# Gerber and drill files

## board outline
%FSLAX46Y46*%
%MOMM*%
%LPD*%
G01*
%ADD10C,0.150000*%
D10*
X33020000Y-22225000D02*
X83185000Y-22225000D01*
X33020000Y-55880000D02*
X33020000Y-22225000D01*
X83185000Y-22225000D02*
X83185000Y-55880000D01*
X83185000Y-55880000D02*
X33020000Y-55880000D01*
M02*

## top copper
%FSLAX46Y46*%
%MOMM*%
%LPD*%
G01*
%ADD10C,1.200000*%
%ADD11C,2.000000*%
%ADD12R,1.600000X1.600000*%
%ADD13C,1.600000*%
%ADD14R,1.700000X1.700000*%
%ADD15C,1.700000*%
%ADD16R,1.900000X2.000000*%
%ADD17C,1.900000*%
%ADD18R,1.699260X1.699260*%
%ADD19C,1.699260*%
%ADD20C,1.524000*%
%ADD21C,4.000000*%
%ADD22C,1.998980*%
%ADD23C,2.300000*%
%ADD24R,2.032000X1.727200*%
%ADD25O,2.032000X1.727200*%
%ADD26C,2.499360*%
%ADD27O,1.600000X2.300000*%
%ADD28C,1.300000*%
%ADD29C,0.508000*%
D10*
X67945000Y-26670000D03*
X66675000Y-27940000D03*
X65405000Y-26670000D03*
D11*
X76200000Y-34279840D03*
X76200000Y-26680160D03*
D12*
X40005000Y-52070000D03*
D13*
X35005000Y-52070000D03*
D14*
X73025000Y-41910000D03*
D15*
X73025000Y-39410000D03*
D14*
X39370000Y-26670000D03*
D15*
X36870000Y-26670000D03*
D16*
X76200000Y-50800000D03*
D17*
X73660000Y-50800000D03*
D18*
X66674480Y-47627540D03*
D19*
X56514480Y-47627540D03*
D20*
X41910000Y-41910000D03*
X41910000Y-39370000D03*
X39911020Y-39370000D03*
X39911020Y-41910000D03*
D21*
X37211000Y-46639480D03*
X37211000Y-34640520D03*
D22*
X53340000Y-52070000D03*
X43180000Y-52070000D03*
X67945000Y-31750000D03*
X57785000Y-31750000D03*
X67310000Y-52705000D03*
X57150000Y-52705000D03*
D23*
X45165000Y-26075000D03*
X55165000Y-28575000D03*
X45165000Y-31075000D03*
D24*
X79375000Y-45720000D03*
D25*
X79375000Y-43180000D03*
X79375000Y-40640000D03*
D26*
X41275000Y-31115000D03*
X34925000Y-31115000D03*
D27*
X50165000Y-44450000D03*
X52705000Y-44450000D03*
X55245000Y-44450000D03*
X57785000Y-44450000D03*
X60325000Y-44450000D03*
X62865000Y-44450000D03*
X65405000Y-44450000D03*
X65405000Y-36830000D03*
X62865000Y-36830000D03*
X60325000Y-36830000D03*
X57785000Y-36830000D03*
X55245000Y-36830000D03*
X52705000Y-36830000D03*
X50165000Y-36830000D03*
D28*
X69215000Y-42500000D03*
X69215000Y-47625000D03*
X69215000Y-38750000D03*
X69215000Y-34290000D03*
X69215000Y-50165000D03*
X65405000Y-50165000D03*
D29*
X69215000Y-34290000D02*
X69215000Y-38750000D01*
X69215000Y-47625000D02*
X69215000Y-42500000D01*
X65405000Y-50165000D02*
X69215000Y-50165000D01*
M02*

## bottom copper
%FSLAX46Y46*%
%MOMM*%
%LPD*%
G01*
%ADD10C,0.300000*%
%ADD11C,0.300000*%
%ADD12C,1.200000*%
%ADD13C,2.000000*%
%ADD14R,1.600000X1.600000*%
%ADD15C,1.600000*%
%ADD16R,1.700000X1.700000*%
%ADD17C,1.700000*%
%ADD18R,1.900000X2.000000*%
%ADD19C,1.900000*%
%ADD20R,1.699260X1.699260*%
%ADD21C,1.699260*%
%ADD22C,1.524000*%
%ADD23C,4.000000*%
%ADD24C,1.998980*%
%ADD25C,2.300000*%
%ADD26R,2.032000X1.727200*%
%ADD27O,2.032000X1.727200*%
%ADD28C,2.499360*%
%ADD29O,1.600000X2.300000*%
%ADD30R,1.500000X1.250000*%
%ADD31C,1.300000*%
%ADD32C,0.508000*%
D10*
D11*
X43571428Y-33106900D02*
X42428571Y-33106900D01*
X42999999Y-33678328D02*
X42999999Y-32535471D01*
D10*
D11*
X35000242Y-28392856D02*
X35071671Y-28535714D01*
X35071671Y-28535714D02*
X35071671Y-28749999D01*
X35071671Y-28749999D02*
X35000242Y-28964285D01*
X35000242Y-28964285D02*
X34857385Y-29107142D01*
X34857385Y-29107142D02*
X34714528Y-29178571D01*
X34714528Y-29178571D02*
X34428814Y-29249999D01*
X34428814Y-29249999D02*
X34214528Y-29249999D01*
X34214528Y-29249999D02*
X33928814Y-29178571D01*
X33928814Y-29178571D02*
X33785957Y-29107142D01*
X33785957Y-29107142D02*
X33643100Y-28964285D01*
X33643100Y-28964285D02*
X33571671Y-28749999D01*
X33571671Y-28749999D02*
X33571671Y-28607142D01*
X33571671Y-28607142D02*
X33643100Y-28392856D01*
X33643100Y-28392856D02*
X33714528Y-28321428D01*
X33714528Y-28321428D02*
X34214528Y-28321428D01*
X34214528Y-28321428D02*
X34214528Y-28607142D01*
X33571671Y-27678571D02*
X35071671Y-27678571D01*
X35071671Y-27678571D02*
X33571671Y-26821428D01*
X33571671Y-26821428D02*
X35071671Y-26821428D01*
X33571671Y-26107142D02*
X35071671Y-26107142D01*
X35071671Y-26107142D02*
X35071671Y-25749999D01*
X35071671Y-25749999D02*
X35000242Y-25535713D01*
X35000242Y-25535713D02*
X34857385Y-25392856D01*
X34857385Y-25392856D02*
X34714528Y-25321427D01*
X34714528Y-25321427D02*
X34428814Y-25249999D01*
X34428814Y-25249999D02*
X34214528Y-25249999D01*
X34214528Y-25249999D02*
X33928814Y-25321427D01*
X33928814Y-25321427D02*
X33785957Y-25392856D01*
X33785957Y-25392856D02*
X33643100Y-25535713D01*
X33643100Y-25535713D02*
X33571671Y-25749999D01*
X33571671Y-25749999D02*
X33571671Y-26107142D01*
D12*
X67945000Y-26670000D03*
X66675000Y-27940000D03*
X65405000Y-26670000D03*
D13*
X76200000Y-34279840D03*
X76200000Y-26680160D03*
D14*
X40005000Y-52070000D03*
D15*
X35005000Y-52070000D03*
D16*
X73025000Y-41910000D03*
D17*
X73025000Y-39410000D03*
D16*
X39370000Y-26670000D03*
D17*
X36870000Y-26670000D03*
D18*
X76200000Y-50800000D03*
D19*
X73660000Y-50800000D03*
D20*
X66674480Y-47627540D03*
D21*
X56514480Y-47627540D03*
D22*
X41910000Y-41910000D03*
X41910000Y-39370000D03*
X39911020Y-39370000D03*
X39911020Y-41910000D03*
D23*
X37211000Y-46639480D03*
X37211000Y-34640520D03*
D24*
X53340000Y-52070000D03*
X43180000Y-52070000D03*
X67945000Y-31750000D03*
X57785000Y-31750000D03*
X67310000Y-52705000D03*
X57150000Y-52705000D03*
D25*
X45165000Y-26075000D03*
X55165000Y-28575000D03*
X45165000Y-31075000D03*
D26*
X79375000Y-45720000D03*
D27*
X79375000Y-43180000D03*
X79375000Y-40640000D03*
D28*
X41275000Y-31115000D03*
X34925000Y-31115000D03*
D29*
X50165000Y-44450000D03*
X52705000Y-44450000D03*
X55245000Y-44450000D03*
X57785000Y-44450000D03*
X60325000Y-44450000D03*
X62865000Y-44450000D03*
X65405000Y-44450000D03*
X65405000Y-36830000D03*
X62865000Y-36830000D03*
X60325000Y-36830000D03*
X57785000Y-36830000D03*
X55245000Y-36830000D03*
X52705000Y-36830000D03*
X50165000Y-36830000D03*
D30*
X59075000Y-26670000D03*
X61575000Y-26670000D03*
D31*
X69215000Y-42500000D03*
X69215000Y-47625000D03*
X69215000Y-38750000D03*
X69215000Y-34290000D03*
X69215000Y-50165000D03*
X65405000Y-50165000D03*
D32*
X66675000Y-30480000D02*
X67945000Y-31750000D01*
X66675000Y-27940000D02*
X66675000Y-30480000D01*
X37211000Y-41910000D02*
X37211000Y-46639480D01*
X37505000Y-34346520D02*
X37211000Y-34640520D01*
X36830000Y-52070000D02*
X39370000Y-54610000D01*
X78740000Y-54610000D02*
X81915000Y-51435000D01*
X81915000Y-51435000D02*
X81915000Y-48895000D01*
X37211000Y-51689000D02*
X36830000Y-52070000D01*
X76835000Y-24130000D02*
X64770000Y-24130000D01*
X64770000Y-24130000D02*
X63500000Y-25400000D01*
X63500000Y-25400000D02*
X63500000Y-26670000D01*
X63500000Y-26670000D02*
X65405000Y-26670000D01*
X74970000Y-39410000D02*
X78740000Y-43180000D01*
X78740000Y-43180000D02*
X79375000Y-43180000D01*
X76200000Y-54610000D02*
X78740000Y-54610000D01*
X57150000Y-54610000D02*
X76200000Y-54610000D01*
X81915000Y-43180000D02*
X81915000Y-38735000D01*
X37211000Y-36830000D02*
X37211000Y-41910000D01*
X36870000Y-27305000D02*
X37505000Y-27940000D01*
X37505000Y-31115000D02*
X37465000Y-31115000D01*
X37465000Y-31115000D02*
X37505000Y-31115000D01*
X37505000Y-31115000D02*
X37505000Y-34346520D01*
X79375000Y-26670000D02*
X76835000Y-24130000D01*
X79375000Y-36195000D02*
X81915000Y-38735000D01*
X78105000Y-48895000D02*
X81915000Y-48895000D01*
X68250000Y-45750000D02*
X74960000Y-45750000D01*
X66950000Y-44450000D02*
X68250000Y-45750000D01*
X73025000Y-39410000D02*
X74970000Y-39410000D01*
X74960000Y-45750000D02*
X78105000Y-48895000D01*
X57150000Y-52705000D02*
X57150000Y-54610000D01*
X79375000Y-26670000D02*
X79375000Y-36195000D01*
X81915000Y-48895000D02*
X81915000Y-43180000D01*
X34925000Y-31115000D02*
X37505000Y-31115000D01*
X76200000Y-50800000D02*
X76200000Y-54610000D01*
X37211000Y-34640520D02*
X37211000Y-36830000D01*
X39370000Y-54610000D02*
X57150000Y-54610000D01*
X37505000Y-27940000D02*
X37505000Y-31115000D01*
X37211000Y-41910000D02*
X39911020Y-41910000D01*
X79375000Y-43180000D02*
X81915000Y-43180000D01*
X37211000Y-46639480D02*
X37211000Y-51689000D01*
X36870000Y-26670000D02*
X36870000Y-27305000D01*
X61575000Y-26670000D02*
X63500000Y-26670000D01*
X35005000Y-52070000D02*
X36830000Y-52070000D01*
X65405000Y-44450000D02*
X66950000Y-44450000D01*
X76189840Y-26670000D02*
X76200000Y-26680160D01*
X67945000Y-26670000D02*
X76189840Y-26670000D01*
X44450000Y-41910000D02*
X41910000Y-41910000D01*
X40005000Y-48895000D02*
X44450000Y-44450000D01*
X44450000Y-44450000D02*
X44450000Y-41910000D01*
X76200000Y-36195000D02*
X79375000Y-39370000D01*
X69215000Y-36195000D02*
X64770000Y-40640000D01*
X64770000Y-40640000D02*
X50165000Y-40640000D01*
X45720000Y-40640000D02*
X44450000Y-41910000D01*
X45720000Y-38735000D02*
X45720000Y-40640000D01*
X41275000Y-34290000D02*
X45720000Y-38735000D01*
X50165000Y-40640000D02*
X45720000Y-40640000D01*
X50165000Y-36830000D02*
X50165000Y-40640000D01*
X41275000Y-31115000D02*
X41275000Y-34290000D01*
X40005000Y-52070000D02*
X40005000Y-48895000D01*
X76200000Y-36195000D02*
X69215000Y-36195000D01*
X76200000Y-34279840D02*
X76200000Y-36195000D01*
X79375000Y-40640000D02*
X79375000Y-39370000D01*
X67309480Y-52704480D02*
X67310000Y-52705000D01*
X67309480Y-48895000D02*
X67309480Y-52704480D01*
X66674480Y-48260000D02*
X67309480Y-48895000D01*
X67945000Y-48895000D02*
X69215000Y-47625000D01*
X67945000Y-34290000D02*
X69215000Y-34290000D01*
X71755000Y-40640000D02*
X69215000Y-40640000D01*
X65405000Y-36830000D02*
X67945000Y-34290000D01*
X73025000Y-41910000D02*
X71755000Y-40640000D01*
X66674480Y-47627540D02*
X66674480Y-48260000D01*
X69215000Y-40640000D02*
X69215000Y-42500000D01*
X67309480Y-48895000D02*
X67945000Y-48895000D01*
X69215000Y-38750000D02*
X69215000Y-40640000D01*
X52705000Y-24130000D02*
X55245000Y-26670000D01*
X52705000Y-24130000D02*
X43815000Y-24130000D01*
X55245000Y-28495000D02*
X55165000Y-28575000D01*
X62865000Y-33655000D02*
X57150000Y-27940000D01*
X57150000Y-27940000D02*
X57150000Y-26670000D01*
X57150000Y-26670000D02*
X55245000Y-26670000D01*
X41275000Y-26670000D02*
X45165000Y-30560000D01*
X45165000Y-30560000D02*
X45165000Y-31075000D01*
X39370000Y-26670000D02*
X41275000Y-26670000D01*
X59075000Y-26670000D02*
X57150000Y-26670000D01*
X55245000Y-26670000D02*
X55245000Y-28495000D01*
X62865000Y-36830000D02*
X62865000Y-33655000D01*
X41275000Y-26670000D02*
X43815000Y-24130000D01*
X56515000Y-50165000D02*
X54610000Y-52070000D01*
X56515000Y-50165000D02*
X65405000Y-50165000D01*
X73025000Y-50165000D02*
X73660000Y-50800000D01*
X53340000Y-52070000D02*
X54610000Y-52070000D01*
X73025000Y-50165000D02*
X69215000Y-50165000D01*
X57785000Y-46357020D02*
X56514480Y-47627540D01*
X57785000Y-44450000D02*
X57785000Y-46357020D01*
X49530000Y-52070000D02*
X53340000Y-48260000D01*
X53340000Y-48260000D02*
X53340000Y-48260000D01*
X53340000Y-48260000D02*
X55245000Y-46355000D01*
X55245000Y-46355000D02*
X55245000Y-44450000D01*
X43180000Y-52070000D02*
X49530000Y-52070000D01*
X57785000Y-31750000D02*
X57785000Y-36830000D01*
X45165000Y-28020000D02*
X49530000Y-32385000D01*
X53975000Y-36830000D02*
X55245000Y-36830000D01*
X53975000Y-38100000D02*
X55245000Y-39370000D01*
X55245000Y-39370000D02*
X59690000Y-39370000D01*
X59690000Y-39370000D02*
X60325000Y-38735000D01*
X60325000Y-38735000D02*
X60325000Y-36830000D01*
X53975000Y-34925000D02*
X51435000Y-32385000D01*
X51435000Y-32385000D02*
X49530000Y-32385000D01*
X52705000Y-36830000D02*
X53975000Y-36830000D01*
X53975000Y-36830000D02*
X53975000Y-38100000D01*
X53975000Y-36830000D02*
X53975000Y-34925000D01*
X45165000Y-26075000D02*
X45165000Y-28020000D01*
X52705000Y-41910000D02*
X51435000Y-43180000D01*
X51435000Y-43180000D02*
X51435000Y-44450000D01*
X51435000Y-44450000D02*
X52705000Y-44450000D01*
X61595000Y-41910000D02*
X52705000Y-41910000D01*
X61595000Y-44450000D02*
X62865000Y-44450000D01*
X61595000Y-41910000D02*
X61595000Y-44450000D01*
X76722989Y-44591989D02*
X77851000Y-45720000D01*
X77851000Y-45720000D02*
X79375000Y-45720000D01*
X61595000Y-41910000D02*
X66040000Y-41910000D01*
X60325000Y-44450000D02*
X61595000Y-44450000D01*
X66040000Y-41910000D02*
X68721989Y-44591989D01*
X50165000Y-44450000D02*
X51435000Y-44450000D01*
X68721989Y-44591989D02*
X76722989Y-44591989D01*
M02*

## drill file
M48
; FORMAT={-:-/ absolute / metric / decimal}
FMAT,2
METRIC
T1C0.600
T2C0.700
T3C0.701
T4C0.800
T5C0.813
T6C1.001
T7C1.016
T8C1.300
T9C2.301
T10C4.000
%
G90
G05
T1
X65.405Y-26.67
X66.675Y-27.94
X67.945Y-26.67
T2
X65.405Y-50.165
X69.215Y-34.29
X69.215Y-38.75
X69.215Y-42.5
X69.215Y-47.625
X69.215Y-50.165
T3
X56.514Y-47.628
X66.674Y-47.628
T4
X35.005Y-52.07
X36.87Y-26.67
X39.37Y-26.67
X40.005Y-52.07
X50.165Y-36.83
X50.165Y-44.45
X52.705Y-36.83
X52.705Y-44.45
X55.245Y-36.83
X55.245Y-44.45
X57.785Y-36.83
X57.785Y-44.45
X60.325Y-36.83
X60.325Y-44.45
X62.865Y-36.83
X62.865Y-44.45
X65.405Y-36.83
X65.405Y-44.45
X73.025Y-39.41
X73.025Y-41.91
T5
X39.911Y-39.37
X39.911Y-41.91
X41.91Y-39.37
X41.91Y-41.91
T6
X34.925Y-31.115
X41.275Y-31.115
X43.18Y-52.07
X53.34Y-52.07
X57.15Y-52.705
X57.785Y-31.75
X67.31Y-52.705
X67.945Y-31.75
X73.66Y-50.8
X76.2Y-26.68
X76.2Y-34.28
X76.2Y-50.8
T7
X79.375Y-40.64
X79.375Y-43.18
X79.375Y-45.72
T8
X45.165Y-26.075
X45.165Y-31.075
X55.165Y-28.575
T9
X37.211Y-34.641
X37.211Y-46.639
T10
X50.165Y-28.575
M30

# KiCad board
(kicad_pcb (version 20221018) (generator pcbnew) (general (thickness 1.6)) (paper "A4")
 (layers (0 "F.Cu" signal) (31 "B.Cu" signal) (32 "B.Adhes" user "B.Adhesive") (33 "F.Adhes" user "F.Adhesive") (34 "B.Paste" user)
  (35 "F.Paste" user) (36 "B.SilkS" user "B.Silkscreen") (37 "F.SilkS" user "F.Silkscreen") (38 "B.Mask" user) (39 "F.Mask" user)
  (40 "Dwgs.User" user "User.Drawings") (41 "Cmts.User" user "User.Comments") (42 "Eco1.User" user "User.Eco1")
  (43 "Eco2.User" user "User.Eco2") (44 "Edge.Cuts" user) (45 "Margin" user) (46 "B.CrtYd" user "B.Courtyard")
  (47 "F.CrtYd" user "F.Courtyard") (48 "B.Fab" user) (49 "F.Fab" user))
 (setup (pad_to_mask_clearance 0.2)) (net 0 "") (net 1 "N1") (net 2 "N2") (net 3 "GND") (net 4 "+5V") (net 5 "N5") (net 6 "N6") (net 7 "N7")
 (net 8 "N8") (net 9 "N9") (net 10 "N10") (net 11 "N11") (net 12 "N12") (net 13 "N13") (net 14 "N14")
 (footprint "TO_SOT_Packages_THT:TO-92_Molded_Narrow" (layer "F.Cu") (at 67.945 26.67 180)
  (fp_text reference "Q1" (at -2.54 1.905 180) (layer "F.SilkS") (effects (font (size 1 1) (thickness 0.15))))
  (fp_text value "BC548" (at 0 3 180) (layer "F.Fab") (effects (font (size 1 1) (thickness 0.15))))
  (pad "1" thru_hole circle (at 0 0 270) (size 1.2 1.2) (drill 0.6) (layers "*.Cu" "*.Mask" "F.SilkS") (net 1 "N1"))
  (pad "2" thru_hole circle (at 1.27 -1.27 270) (size 1.2 1.2) (drill 0.6) (layers "*.Cu" "*.Mask" "F.SilkS") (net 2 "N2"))
  (pad "3" thru_hole circle (at 2.54 0 270) (size 1.2 1.2) (drill 0.6) (layers "*.Cu" "*.Mask" "F.SilkS") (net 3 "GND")))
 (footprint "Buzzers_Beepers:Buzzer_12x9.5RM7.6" (layer "F.Cu") (at 76.2 30.48 90)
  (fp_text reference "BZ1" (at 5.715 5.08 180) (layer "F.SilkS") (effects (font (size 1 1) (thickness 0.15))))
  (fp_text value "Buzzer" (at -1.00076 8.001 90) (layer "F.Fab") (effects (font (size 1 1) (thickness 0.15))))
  (pad "1" thru_hole circle (at -3.79984 0 90) (size 2 2) (drill 1.00076) (layers "*.Cu" "*.Mask" "F.SilkS") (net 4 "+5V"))
  (pad "2" thru_hole circle (at 3.79984 0 90) (size 2 2) (drill 1.00076) (layers "*.Cu" "*.Mask" "F.SilkS") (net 1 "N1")))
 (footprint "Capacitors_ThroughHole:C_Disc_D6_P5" (layer "F.Cu") (at 40.005 52.07 180)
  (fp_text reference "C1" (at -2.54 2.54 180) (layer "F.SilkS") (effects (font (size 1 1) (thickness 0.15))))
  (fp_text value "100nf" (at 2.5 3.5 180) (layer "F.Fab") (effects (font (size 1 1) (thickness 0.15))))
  (pad "1" thru_hole rect (at 0 0 180) (size 1.6 1.6) (drill 0.8) (layers "*.Cu" "*.Mask" "F.SilkS") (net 4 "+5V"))
  (pad "2" thru_hole circle (at 5 0 180) (size 1.6 1.6) (drill 0.8) (layers "*.Cu" "*.Mask" "F.SilkS") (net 3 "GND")))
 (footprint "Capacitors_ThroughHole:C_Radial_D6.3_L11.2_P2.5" (layer "F.Cu") (at 73.025 41.91 90)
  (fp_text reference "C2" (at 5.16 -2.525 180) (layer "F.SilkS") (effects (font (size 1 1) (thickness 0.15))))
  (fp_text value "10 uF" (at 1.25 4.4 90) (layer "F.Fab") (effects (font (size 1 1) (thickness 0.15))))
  (pad "1" thru_hole rect (at 0 0 90) (size 1.7 1.7) (drill 0.8) (layers "*.Cu" "*.Mask" "F.SilkS") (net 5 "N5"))
  (pad "2" thru_hole circle (at 2.5 0 90) (size 1.7 1.7) (drill 0.8) (layers "*.Cu" "*.Mask" "F.SilkS") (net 3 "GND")))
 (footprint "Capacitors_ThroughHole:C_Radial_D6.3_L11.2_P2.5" (layer "F.Cu") (at 39.37 26.67 180)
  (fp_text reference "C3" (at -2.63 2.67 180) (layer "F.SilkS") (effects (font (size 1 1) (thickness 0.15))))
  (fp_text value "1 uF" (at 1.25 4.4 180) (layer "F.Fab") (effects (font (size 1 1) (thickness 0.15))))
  (pad "1" thru_hole rect (at 0 0 180) (size 1.7 1.7) (drill 0.8) (layers "*.Cu" "*.Mask" "F.SilkS") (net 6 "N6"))
  (pad "2" thru_hole circle (at 2.5 0 180) (size 1.7 1.7) (drill 0.8) (layers "*.Cu" "*.Mask" "F.SilkS") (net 3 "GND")))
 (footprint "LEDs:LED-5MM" (layer "F.Cu") (at 76.2 50.8 180)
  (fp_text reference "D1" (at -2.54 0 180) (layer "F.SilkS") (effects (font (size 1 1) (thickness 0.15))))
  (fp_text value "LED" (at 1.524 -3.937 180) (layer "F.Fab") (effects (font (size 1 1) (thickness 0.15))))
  (pad "1" thru_hole rect (at 0 0 270) (size 2 1.9) (drill 1.00076) (layers "*.Cu" "*.Mask" "F.SilkS") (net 3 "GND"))
  (pad "2" thru_hole circle (at 2.54 0 180) (size 1.9 1.9) (drill 1.00076) (layers "*.Cu" "*.Mask" "F.SilkS") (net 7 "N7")))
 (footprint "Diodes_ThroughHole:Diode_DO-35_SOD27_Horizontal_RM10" (layer "F.Cu") (at 66.675 47.625 180)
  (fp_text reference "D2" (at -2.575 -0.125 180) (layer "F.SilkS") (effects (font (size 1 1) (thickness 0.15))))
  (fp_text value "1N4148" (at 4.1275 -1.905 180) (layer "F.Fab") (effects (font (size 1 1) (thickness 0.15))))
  (pad "1" thru_hole rect (at 0.00052 -0.00254) (size 1.69926 1.69926) (drill 0.70104) (layers "*.Cu" "*.Mask" "F.SilkS") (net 5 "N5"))
  (pad "2" thru_hole circle (at 10.16052 -0.00254) (size 1.69926 1.69926) (drill 0.70104) (layers "*.Cu" "*.Mask" "F.SilkS") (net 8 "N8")))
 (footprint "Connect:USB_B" (layer "F.Cu") (at 41.91 41.91 180) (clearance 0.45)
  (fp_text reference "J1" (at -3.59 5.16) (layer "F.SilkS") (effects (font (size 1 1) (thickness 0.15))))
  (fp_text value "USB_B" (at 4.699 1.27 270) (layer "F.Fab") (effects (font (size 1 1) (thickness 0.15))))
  (pad "1" thru_hole circle (at 0 0 90) (size 1.524 1.524) (drill 0.8128) (layers "*.Cu" "*.Mask" "F.SilkS") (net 4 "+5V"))
  (pad "2" thru_hole circle (at 0 2.54 90) (size 1.524 1.524) (drill 0.8128) (layers "*.Cu" "*.Mask" "F.SilkS") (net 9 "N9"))
  (pad "3" thru_hole circle (at 1.99898 2.54 90) (size 1.524 1.524) (drill 0.8128) (layers "*.Cu" "*.Mask" "F.SilkS") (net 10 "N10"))
  (pad "4" thru_hole circle (at 1.99898 0 90) (size 1.524 1.524) (drill 0.8128) (layers "*.Cu" "*.Mask" "F.SilkS") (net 3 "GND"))
  (pad "5" thru_hole circle (at 4.699 -4.72948 90) (size 4 4) (drill 2.30124) (layers "*.Cu" "*.Mask" "F.SilkS") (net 3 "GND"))
  (pad "5" thru_hole circle (at 4.699 7.26948 90) (size 4 4) (drill 2.30124) (layers "*.Cu" "*.Mask" "F.SilkS") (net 3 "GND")))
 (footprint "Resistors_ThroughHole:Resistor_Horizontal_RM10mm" (layer "F.Cu") (at 53.34 52.07 180)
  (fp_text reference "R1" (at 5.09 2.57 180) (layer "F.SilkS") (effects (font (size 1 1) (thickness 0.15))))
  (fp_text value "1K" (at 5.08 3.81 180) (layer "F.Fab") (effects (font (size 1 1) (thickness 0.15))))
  (pad "1" thru_hole circle (at 0 0 180) (size 1.99898 1.99898) (drill 1.00076) (layers "*.Cu" "*.SilkS" "*.Mask") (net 7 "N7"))
  (pad "2" thru_hole circle (at 10.16 0 180) (size 1.99898 1.99898) (drill 1.00076) (layers "*.Cu" "*.SilkS" "*.Mask") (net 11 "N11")))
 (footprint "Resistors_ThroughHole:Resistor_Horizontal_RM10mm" (layer "F.Cu") (at 67.945 31.75 180)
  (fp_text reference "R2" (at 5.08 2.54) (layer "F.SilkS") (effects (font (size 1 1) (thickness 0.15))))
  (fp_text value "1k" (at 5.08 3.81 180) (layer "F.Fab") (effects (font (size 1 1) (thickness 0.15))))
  (pad "1" thru_hole circle (at 0 0 180) (size 1.99898 1.99898) (drill 1.00076) (layers "*.Cu" "*.SilkS" "*.Mask") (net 2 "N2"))
  (pad "2" thru_hole circle (at 10.16 0 180) (size 1.99898 1.99898) (drill 1.00076) (layers "*.Cu" "*.SilkS" "*.Mask") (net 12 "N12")))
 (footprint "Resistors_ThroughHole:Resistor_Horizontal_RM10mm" (layer "F.Cu") (at 67.31 52.705 180)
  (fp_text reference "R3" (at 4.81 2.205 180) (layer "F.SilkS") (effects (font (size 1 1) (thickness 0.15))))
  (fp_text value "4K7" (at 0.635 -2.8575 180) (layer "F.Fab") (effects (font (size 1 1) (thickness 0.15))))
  (pad "1" thru_hole circle (at 0 0 180) (size 1.99898 1.99898) (drill 1.00076) (layers "*.Cu" "*.SilkS" "*.Mask") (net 5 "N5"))
  (pad "2" thru_hole circle (at 10.16 0 180) (size 1.99898 1.99898) (drill 1.00076) (layers "*.Cu" "*.SilkS" "*.Mask") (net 3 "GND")))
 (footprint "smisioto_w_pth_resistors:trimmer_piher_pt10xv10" (layer "F.Cu") (at 50.165 28.575 90)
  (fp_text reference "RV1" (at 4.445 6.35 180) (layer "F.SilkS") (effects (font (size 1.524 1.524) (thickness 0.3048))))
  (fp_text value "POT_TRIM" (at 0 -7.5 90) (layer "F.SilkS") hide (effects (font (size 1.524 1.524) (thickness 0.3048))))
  (pad "" np_thru_hole circle (at 0 0 90) (size 4 4) (drill 4) (layers "*.Cu" "*.Mask" "F.SilkS"))
  (pad "1" thru_hole circle (at 2.5 -5 90) (size 2.3 2.3) (drill 1.3) (layers "*.Cu" "*.Mask" "F.SilkS") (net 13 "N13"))
  (pad "2" thru_hole circle (at 0 5 90) (size 2.3 2.3) (drill 1.3) (layers "*.Cu" "*.Mask" "F.SilkS") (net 6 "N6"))
  (pad "3" thru_hole circle (at -2.5 -5 90) (size 2.3 2.3) (drill 1.3) (layers "*.Cu" "*.Mask" "F.SilkS") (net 6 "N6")))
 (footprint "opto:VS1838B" (layer "F.Cu") (at 79.375 45.72 180)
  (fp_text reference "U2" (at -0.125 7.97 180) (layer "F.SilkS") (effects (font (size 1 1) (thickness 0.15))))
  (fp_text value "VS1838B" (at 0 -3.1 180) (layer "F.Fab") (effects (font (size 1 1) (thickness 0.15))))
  (pad "1" thru_hole rect (at 0 0 180) (size 2.032 1.7272) (drill 1.016) (layers "*.Cu" "*.Mask" "F.SilkS") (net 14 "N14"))
  (pad "2" thru_hole oval (at 0 2.54 180) (size 2.032 1.7272) (drill 1.016) (layers "*.Cu" "*.Mask" "F.SilkS") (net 3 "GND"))
  (pad "3" thru_hole oval (at 0 5.08 180) (size 2.032 1.7272) (drill 1.016) (layers "*.Cu" "*.Mask" "F.SilkS") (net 4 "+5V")))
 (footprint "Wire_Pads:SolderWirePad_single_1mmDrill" (layer "F.Cu") (at 41.275 31.115)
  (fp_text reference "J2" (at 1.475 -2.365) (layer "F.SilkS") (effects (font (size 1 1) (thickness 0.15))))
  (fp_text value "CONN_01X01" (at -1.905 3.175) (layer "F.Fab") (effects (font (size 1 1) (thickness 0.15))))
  (pad "1" thru_hole circle (at 0 0) (size 2.49936 2.49936) (drill 1.00076) (layers "*.Cu" "*.Mask" "F.SilkS") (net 4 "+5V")))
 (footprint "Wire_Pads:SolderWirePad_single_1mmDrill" (layer "F.Cu") (at 34.925 31.115)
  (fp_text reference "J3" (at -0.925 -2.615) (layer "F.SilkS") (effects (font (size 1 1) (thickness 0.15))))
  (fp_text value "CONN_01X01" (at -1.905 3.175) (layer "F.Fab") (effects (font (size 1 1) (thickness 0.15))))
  (pad "1" thru_hole circle (at 0 0) (size 2.49936 2.49936) (drill 1.00076) (layers "*.Cu" "*.Mask" "F.SilkS") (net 3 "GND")))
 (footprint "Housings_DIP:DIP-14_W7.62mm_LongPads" (layer "F.Cu") (at 50.165 44.45 90)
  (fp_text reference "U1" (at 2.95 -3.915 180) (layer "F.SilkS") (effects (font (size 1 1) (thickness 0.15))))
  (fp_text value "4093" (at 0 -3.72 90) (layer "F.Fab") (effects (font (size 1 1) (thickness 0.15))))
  (pad "1" thru_hole oval (at 0 0 90) (size 2.3 1.6) (drill 0.8) (layers "*.Cu" "*.Mask" "F.SilkS") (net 14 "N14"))
  (pad "2" thru_hole oval (at 0 2.54 90) (size 2.3 1.6) (drill 0.8) (layers "*.Cu" "*.Mask" "F.SilkS") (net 14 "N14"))
  (pad "3" thru_hole oval (at 0 5.08 90) (size 2.3 1.6) (drill 0.8) (layers "*.Cu" "*.Mask" "F.SilkS") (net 11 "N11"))
  (pad "4" thru_hole oval (at 0 7.62 90) (size 2.3 1.6) (drill 0.8) (layers "*.Cu" "*.Mask" "F.SilkS") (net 8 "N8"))
  (pad "5" thru_hole oval (at 0 10.16 90) (size 2.3 1.6) (drill 0.8) (layers "*.Cu" "*.Mask" "F.SilkS") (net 14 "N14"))
  (pad "6" thru_hole oval (at 0 12.7 90) (size 2.3 1.6) (drill 0.8) (layers "*.Cu" "*.Mask" "F.SilkS") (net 14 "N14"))
  (pad "7" thru_hole oval (at 0 15.24 90) (size 2.3 1.6) (drill 0.8) (layers "*.Cu" "*.Mask" "F.SilkS") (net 3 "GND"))
  (pad "8" thru_hole oval (at 7.62 15.24 90) (size 2.3 1.6) (drill 0.8) (layers "*.Cu" "*.Mask" "F.SilkS") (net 5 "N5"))
  (pad "9" thru_hole oval (at 7.62 12.7 90) (size 2.3 1.6) (drill 0.8) (layers "*.Cu" "*.Mask" "F.SilkS") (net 6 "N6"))
  (pad "10" thru_hole oval (at 7.62 10.16 90) (size 2.3 1.6) (drill 0.8) (layers "*.Cu" "*.Mask" "F.SilkS") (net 13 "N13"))
  (pad "11" thru_hole oval (at 7.62 7.62 90) (size 2.3 1.6) (drill 0.8) (layers "*.Cu" "*.Mask" "F.SilkS") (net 12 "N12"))
  (pad "12" thru_hole oval (at 7.62 5.08 90) (size 2.3 1.6) (drill 0.8) (layers "*.Cu" "*.Mask" "F.SilkS") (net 13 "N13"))
  (pad "13" thru_hole oval (at 7.62 2.54 90) (size 2.3 1.6) (drill 0.8) (layers "*.Cu" "*.Mask" "F.SilkS") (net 13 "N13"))
  (pad "14" thru_hole oval (at 7.62 0 90) (size 2.3 1.6) (drill 0.8) (layers "*.Cu" "*.Mask" "F.SilkS") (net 4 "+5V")))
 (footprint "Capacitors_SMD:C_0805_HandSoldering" (layer "B.Cu") (at 60.325 26.67)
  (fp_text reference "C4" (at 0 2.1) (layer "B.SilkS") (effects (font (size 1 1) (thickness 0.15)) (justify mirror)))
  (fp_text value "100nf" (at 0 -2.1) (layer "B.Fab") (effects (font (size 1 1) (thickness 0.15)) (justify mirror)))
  (pad "1" smd rect (at -1.25 0) (size 1.5 1.25) (layers "B.Cu" "B.Paste" "B.Mask") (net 6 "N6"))
  (pad "2" smd rect (at 1.25 0) (size 1.5 1.25) (layers "B.Cu" "B.Paste" "B.Mask") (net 3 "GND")))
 (gr_line (start 33.02 22.225) (end 83.185 22.225) (stroke (width 0.15) (type solid)) (layer "Edge.Cuts"))
 (gr_line (start 33.02 55.88) (end 33.02 22.225) (stroke (width 0.15) (type solid)) (layer "Edge.Cuts"))
 (gr_line (start 83.185 22.225) (end 83.185 55.88) (stroke (width 0.15) (type solid)) (layer "Edge.Cuts"))
 (gr_line (start 83.185 55.88) (end 33.02 55.88) (stroke (width 0.15) (type solid)) (layer "Edge.Cuts"))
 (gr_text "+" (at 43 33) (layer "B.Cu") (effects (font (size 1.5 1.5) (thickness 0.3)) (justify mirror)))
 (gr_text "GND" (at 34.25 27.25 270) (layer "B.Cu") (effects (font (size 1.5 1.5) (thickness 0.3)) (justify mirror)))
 (segment (start 66.675 30.48) (end 67.945 31.75) (width 0.508) (layer "B.Cu") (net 2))
 (segment (start 66.675 27.94) (end 66.675 30.48) (width 0.508) (layer "B.Cu") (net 2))
 (segment (start 37.211 41.91) (end 37.211 46.63948) (width 0.508) (layer "B.Cu") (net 3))
 (segment (start 37.505 34.34652) (end 37.211 34.64052) (width 0.508) (layer "B.Cu") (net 3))
 (segment (start 36.83 52.07) (end 39.37 54.61) (width 0.508) (layer "B.Cu") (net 3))
 (segment (start 78.74 54.61) (end 81.915 51.435) (width 0.508) (layer "B.Cu") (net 3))
 (segment (start 81.915 51.435) (end 81.915 48.895) (width 0.508) (layer "B.Cu") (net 3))
 (segment (start 37.211 51.689) (end 36.83 52.07) (width 0.508) (layer "B.Cu") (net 3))
 (segment (start 76.835 24.13) (end 64.77 24.13) (width 0.508) (layer "B.Cu") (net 3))
 (segment (start 64.77 24.13) (end 63.5 25.4) (width 0.508) (layer "B.Cu") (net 3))
 (segment (start 63.5 25.4) (end 63.5 26.67) (width 0.508) (layer "B.Cu") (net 3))
 (segment (start 63.5 26.67) (end 65.405 26.67) (width 0.508) (layer "B.Cu") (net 3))
 (segment (start 74.97 39.41) (end 78.74 43.18) (width 0.508) (layer "B.Cu") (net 3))
 (segment (start 78.74 43.18) (end 79.375 43.18) (width 0.508) (layer "B.Cu") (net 3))
 (segment (start 76.2 54.61) (end 78.74 54.61) (width 0.508) (layer "B.Cu") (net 3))
 (segment (start 57.15 54.61) (end 76.2 54.61) (width 0.508) (layer "B.Cu") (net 3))
 (segment (start 81.915 43.18) (end 81.915 38.735) (width 0.508) (layer "B.Cu") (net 3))
 (segment (start 37.211 36.83) (end 37.211 41.91) (width 0.508) (layer "B.Cu") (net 3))
 (segment (start 36.87 27.305) (end 37.505 27.94) (width 0.508) (layer "B.Cu") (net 3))
 (segment (start 37.505 31.115) (end 37.465 31.115) (width 0.508) (layer "B.Cu") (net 3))
 (segment (start 37.465 31.115) (end 37.505 31.115) (width 0.508) (layer "B.Cu") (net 3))
 (segment (start 37.505 31.115) (end 37.505 34.34652) (width 0.508) (layer "B.Cu") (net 3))
 (segment (start 79.375 26.67) (end 76.835 24.13) (width 0.508) (layer "B.Cu") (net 3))
 (segment (start 79.375 36.195) (end 81.915 38.735) (width 0.508) (layer "B.Cu") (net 3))
 (segment (start 78.105 48.895) (end 81.915 48.895) (width 0.508) (layer "B.Cu") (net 3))
 (segment (start 68.25 45.75) (end 74.96 45.75) (width 0.508) (layer "B.Cu") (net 3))
 (segment (start 66.95 44.45) (end 68.25 45.75) (width 0.508) (layer "B.Cu") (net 3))
 (segment (start 73.025 39.41) (end 74.97 39.41) (width 0.508) (layer "B.Cu") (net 3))
 (segment (start 74.96 45.75) (end 78.105 48.895) (width 0.508) (layer "B.Cu") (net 3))
 (segment (start 57.15 52.705) (end 57.15 54.61) (width 0.508) (layer "B.Cu") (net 3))
 (segment (start 79.375 26.67) (end 79.375 36.195) (width 0.508) (layer "B.Cu") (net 3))
 (segment (start 81.915 48.895) (end 81.915 43.18) (width 0.508) (layer "B.Cu") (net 3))
 (segment (start 34.925 31.115) (end 37.505 31.115) (width 0.508) (layer "B.Cu") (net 3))
 (segment (start 76.2 50.8) (end 76.2 54.61) (width 0.508) (layer "B.Cu") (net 3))
 (segment (start 37.211 34.64052) (end 37.211 36.83) (width 0.508) (layer "B.Cu") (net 3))
 (segment (start 39.37 54.61) (end 57.15 54.61) (width 0.508) (layer "B.Cu") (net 3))
 (segment (start 37.505 27.94) (end 37.505 31.115) (width 0.508) (layer "B.Cu") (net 3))
 (segment (start 37.211 41.91) (end 39.91102 41.91) (width 0.508) (layer "B.Cu") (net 3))
 (segment (start 79.375 43.18) (end 81.915 43.18) (width 0.508) (layer "B.Cu") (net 3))
 (segment (start 37.211 46.63948) (end 37.211 51.689) (width 0.508) (layer "B.Cu") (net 3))
 (segment (start 36.87 26.67) (end 36.87 27.305) (width 0.508) (layer "B.Cu") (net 3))
 (segment (start 61.575 26.67) (end 63.5 26.67) (width 0.508) (layer "B.Cu") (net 3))
 (segment (start 35.005 52.07) (end 36.83 52.07) (width 0.508) (layer "B.Cu") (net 3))
 (segment (start 65.405 44.45) (end 66.95 44.45) (width 0.508) (layer "B.Cu") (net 3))
 (segment (start 76.18984 26.67) (end 76.2 26.68016) (width 0.508) (layer "B.Cu") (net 1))
 (segment (start 67.945 26.67) (end 76.18984 26.67) (width 0.508) (layer "B.Cu") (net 1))
 (segment (start 44.45 41.91) (end 41.91 41.91) (width 0.508) (layer "B.Cu") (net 4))
 (segment (start 40.005 48.895) (end 44.45 44.45) (width 0.508) (layer "B.Cu") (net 4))
 (segment (start 44.45 44.45) (end 44.45 41.91) (width 0.508) (layer "B.Cu") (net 4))
 (segment (start 76.2 36.195) (end 79.375 39.37) (width 0.508) (layer "B.Cu") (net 4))
 (segment (start 69.215 36.195) (end 64.77 40.64) (width 0.508) (layer "B.Cu") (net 4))
 (segment (start 64.77 40.64) (end 50.165 40.64) (width 0.508) (layer "B.Cu") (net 4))
 (segment (start 45.72 40.64) (end 44.45 41.91) (width 0.508) (layer "B.Cu") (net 4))
 (segment (start 45.72 38.735) (end 45.72 40.64) (width 0.508) (layer "B.Cu") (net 4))
 (segment (start 41.275 34.29) (end 45.72 38.735) (width 0.508) (layer "B.Cu") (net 4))
 (segment (start 50.165 40.64) (end 45.72 40.64) (width 0.508) (layer "B.Cu") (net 4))
 (segment (start 50.165 36.83) (end 50.165 40.64) (width 0.508) (layer "B.Cu") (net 4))
 (segment (start 41.275 31.115) (end 41.275 34.29) (width 0.508) (layer "B.Cu") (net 4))
 (segment (start 40.005 52.07) (end 40.005 48.895) (width 0.508) (layer "B.Cu") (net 4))
 (segment (start 76.2 36.195) (end 69.215 36.195) (width 0.508) (layer "B.Cu") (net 4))
 (segment (start 76.2 34.27984) (end 76.2 36.195) (width 0.508) (layer "B.Cu") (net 4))
 (segment (start 79.375 40.64) (end 79.375 39.37) (width 0.508) (layer "B.Cu") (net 4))
 (segment (start 69.215 34.29) (end 69.215 38.75) (width 0.508) (layer "F.Cu") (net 5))
 (segment (start 69.215 47.625) (end 69.215 42.5) (width 0.508) (layer "F.Cu") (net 5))
 (via (at 69.215 42.5) (size 1.3) (drill 0.7) (layers "F.Cu" "B.Cu") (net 5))
 (via (at 69.215 47.625) (size 1.3) (drill 0.7) (layers "F.Cu" "B.Cu") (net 5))
 (via (at 69.215 38.75) (size 1.3) (drill 0.7) (layers "F.Cu" "B.Cu") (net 5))
 (via (at 69.215 34.29) (size 1.3) (drill 0.7) (layers "F.Cu" "B.Cu") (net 5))
 (segment (start 67.30948 52.70448) (end 67.31 52.705) (width 0.508) (layer "B.Cu") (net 5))
 (segment (start 67.30948 48.895) (end 67.30948 52.70448) (width 0.508) (layer "B.Cu") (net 5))
 (segment (start 66.67448 48.26) (end 67.30948 48.895) (width 0.508) (layer "B.Cu") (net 5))
 (segment (start 67.945 48.895) (end 69.215 47.625) (width 0.508) (layer "B.Cu") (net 5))
 (segment (start 67.945 34.29) (end 69.215 34.29) (width 0.508) (layer "B.Cu") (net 5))
 (segment (start 71.755 40.64) (end 69.215 40.64) (width 0.508) (layer "B.Cu") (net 5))
 (segment (start 65.405 36.83) (end 67.945 34.29) (width 0.508) (layer "B.Cu") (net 5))
 (segment (start 73.025 41.91) (end 71.755 40.64) (width 0.508) (layer "B.Cu") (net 5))
 (segment (start 66.67448 47.62754) (end 66.67448 48.26) (width 0.508) (layer "B.Cu") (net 5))
 (segment (start 69.215 40.64) (end 69.215 42.5) (width 0.508) (layer "B.Cu") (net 5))
 (segment (start 67.30948 48.895) (end 67.945 48.895) (width 0.508) (layer "B.Cu") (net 5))
 (segment (start 69.215 38.75) (end 69.215 40.64) (width 0.508) (layer "B.Cu") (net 5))
 (segment (start 52.705 24.13) (end 55.245 26.67) (width 0.508) (layer "B.Cu") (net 6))
 (segment (start 52.705 24.13) (end 43.815 24.13) (width 0.508) (layer "B.Cu") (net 6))
 (segment (start 55.245 28.495) (end 55.165 28.575) (width 0.508) (layer "B.Cu") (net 6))
 (segment (start 62.865 33.655) (end 57.15 27.94) (width 0.508) (layer "B.Cu") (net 6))
 (segment (start 57.15 27.94) (end 57.15 26.67) (width 0.508) (layer "B.Cu") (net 6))
 (segment (start 57.15 26.67) (end 55.245 26.67) (width 0.508) (layer "B.Cu") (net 6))
 (segment (start 41.275 26.67) (end 45.165 30.56) (width 0.508) (layer "B.Cu") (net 6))
 (segment (start 45.165 30.56) (end 45.165 31.075) (width 0.508) (layer "B.Cu") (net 6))
 (segment (start 39.37 26.67) (end 41.275 26.67) (width 0.508) (layer "B.Cu") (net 6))
 (segment (start 59.075 26.67) (end 57.15 26.67) (width 0.508) (layer "B.Cu") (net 6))
 (segment (start 55.245 26.67) (end 55.245 28.495) (width 0.508) (layer "B.Cu") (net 6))
 (segment (start 62.865 36.83) (end 62.865 33.655) (width 0.508) (layer "B.Cu") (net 6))
 (segment (start 41.275 26.67) (end 43.815 24.13) (width 0.508) (layer "B.Cu") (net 6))
 (segment (start 65.405 50.165) (end 69.215 50.165) (width 0.508) (layer "F.Cu") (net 7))
 (via (at 69.215 50.165) (size 1.3) (drill 0.7) (layers "F.Cu" "B.Cu") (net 7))
 (via (at 65.405 50.165) (size 1.3) (drill 0.7) (layers "F.Cu" "B.Cu") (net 7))
 (segment (start 56.515 50.165) (end 54.61 52.07) (width 0.508) (layer "B.Cu") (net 7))
 (segment (start 56.515 50.165) (end 65.405 50.165) (width 0.508) (layer "B.Cu") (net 7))
 (segment (start 73.025 50.165) (end 73.66 50.8) (width 0.508) (layer "B.Cu") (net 7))
 (segment (start 53.34 52.07) (end 54.61 52.07) (width 0.508) (layer "B.Cu") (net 7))
 (segment (start 73.025 50.165) (end 69.215 50.165) (width 0.508) (layer "B.Cu") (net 7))
 (segment (start 57.785 46.35702) (end 56.51448 47.62754) (width 0.508) (layer "B.Cu") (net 8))
 (segment (start 57.785 44.45) (end 57.785 46.35702) (width 0.508) (layer "B.Cu") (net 8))
 (segment (start 49.53 52.07) (end 53.34 48.26) (width 0.508) (layer "B.Cu") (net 11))
 (segment (start 53.34 48.26) (end 53.34 48.26) (width 0.508) (layer "B.Cu") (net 11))
 (segment (start 53.34 48.26) (end 55.245 46.355) (width 0.508) (layer "B.Cu") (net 11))
 (segment (start 55.245 46.355) (end 55.245 44.45) (width 0.508) (layer "B.Cu") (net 11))
 (segment (start 43.18 52.07) (end 49.53 52.07) (width 0.508) (layer "B.Cu") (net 11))
 (segment (start 57.785 31.75) (end 57.785 36.83) (width 0.508) (layer "B.Cu") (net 12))
 (segment (start 45.165 28.02) (end 49.53 32.385) (width 0.508) (layer "B.Cu") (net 13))
 (segment (start 53.975 36.83) (end 55.245 36.83) (width 0.508) (layer "B.Cu") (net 13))
 (segment (start 53.975 38.1) (end 55.245 39.37) (width 0.508) (layer "B.Cu") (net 13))
 (segment (start 55.245 39.37) (end 59.69 39.37) (width 0.508) (layer "B.Cu") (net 13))
 (segment (start 59.69 39.37) (end 60.325 38.735) (width 0.508) (layer "B.Cu") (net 13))
 (segment (start 60.325 38.735) (end 60.325 36.83) (width 0.508) (layer "B.Cu") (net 13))
 (segment (start 53.975 34.925) (end 51.435 32.385) (width 0.508) (layer "B.Cu") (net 13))
 (segment (start 51.435 32.385) (end 49.53 32.385) (width 0.508) (layer "B.Cu") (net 13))
 (segment (start 52.705 36.83) (end 53.975 36.83) (width 0.508) (layer "B.Cu") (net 13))
 (segment (start 53.975 36.83) (end 53.975 38.1) (width 0.508) (layer "B.Cu") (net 13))
 (segment (start 53.975 36.83) (end 53.975 34.925) (width 0.508) (layer "B.Cu") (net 13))
 (segment (start 45.165 26.075) (end 45.165 28.02) (width 0.508) (layer "B.Cu") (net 13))
 (segment (start 52.705 41.91) (end 51.435 43.18) (width 0.508) (layer "B.Cu") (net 14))
 (segment (start 51.435 43.18) (end 51.435 44.45) (width 0.508) (layer "B.Cu") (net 14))
 (segment (start 51.435 44.45) (end 52.705 44.45) (width 0.508) (layer "B.Cu") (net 14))
 (segment (start 61.595 41.91) (end 52.705 41.91) (width 0.508) (layer "B.Cu") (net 14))
 (segment (start 61.595 44.45) (end 62.865 44.45) (width 0.508) (layer "B.Cu") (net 14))
 (segment (start 61.595 41.91) (end 61.595 44.45) (width 0.508) (layer "B.Cu") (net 14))
 (segment (start 76.722989 44.591989) (end 77.851 45.72) (width 0.508) (layer "B.Cu") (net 14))
 (segment (start 77.851 45.72) (end 79.375 45.72) (width 0.508) (layer "B.Cu") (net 14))
 (segment (start 61.595 41.91) (end 66.04 41.91) (width 0.508) (layer "B.Cu") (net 14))
 (segment (start 60.325 44.45) (end 61.595 44.45) (width 0.508) (layer "B.Cu") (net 14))
 (segment (start 66.04 41.91) (end 68.721989 44.591989) (width 0.508) (layer "B.Cu") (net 14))
 (segment (start 50.165 44.45) (end 51.435 44.45) (width 0.508) (layer "B.Cu") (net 14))
 (segment (start 68.721989 44.591989) (end 76.722989 44.591989) (width 0.508) (layer "B.Cu") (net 14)))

